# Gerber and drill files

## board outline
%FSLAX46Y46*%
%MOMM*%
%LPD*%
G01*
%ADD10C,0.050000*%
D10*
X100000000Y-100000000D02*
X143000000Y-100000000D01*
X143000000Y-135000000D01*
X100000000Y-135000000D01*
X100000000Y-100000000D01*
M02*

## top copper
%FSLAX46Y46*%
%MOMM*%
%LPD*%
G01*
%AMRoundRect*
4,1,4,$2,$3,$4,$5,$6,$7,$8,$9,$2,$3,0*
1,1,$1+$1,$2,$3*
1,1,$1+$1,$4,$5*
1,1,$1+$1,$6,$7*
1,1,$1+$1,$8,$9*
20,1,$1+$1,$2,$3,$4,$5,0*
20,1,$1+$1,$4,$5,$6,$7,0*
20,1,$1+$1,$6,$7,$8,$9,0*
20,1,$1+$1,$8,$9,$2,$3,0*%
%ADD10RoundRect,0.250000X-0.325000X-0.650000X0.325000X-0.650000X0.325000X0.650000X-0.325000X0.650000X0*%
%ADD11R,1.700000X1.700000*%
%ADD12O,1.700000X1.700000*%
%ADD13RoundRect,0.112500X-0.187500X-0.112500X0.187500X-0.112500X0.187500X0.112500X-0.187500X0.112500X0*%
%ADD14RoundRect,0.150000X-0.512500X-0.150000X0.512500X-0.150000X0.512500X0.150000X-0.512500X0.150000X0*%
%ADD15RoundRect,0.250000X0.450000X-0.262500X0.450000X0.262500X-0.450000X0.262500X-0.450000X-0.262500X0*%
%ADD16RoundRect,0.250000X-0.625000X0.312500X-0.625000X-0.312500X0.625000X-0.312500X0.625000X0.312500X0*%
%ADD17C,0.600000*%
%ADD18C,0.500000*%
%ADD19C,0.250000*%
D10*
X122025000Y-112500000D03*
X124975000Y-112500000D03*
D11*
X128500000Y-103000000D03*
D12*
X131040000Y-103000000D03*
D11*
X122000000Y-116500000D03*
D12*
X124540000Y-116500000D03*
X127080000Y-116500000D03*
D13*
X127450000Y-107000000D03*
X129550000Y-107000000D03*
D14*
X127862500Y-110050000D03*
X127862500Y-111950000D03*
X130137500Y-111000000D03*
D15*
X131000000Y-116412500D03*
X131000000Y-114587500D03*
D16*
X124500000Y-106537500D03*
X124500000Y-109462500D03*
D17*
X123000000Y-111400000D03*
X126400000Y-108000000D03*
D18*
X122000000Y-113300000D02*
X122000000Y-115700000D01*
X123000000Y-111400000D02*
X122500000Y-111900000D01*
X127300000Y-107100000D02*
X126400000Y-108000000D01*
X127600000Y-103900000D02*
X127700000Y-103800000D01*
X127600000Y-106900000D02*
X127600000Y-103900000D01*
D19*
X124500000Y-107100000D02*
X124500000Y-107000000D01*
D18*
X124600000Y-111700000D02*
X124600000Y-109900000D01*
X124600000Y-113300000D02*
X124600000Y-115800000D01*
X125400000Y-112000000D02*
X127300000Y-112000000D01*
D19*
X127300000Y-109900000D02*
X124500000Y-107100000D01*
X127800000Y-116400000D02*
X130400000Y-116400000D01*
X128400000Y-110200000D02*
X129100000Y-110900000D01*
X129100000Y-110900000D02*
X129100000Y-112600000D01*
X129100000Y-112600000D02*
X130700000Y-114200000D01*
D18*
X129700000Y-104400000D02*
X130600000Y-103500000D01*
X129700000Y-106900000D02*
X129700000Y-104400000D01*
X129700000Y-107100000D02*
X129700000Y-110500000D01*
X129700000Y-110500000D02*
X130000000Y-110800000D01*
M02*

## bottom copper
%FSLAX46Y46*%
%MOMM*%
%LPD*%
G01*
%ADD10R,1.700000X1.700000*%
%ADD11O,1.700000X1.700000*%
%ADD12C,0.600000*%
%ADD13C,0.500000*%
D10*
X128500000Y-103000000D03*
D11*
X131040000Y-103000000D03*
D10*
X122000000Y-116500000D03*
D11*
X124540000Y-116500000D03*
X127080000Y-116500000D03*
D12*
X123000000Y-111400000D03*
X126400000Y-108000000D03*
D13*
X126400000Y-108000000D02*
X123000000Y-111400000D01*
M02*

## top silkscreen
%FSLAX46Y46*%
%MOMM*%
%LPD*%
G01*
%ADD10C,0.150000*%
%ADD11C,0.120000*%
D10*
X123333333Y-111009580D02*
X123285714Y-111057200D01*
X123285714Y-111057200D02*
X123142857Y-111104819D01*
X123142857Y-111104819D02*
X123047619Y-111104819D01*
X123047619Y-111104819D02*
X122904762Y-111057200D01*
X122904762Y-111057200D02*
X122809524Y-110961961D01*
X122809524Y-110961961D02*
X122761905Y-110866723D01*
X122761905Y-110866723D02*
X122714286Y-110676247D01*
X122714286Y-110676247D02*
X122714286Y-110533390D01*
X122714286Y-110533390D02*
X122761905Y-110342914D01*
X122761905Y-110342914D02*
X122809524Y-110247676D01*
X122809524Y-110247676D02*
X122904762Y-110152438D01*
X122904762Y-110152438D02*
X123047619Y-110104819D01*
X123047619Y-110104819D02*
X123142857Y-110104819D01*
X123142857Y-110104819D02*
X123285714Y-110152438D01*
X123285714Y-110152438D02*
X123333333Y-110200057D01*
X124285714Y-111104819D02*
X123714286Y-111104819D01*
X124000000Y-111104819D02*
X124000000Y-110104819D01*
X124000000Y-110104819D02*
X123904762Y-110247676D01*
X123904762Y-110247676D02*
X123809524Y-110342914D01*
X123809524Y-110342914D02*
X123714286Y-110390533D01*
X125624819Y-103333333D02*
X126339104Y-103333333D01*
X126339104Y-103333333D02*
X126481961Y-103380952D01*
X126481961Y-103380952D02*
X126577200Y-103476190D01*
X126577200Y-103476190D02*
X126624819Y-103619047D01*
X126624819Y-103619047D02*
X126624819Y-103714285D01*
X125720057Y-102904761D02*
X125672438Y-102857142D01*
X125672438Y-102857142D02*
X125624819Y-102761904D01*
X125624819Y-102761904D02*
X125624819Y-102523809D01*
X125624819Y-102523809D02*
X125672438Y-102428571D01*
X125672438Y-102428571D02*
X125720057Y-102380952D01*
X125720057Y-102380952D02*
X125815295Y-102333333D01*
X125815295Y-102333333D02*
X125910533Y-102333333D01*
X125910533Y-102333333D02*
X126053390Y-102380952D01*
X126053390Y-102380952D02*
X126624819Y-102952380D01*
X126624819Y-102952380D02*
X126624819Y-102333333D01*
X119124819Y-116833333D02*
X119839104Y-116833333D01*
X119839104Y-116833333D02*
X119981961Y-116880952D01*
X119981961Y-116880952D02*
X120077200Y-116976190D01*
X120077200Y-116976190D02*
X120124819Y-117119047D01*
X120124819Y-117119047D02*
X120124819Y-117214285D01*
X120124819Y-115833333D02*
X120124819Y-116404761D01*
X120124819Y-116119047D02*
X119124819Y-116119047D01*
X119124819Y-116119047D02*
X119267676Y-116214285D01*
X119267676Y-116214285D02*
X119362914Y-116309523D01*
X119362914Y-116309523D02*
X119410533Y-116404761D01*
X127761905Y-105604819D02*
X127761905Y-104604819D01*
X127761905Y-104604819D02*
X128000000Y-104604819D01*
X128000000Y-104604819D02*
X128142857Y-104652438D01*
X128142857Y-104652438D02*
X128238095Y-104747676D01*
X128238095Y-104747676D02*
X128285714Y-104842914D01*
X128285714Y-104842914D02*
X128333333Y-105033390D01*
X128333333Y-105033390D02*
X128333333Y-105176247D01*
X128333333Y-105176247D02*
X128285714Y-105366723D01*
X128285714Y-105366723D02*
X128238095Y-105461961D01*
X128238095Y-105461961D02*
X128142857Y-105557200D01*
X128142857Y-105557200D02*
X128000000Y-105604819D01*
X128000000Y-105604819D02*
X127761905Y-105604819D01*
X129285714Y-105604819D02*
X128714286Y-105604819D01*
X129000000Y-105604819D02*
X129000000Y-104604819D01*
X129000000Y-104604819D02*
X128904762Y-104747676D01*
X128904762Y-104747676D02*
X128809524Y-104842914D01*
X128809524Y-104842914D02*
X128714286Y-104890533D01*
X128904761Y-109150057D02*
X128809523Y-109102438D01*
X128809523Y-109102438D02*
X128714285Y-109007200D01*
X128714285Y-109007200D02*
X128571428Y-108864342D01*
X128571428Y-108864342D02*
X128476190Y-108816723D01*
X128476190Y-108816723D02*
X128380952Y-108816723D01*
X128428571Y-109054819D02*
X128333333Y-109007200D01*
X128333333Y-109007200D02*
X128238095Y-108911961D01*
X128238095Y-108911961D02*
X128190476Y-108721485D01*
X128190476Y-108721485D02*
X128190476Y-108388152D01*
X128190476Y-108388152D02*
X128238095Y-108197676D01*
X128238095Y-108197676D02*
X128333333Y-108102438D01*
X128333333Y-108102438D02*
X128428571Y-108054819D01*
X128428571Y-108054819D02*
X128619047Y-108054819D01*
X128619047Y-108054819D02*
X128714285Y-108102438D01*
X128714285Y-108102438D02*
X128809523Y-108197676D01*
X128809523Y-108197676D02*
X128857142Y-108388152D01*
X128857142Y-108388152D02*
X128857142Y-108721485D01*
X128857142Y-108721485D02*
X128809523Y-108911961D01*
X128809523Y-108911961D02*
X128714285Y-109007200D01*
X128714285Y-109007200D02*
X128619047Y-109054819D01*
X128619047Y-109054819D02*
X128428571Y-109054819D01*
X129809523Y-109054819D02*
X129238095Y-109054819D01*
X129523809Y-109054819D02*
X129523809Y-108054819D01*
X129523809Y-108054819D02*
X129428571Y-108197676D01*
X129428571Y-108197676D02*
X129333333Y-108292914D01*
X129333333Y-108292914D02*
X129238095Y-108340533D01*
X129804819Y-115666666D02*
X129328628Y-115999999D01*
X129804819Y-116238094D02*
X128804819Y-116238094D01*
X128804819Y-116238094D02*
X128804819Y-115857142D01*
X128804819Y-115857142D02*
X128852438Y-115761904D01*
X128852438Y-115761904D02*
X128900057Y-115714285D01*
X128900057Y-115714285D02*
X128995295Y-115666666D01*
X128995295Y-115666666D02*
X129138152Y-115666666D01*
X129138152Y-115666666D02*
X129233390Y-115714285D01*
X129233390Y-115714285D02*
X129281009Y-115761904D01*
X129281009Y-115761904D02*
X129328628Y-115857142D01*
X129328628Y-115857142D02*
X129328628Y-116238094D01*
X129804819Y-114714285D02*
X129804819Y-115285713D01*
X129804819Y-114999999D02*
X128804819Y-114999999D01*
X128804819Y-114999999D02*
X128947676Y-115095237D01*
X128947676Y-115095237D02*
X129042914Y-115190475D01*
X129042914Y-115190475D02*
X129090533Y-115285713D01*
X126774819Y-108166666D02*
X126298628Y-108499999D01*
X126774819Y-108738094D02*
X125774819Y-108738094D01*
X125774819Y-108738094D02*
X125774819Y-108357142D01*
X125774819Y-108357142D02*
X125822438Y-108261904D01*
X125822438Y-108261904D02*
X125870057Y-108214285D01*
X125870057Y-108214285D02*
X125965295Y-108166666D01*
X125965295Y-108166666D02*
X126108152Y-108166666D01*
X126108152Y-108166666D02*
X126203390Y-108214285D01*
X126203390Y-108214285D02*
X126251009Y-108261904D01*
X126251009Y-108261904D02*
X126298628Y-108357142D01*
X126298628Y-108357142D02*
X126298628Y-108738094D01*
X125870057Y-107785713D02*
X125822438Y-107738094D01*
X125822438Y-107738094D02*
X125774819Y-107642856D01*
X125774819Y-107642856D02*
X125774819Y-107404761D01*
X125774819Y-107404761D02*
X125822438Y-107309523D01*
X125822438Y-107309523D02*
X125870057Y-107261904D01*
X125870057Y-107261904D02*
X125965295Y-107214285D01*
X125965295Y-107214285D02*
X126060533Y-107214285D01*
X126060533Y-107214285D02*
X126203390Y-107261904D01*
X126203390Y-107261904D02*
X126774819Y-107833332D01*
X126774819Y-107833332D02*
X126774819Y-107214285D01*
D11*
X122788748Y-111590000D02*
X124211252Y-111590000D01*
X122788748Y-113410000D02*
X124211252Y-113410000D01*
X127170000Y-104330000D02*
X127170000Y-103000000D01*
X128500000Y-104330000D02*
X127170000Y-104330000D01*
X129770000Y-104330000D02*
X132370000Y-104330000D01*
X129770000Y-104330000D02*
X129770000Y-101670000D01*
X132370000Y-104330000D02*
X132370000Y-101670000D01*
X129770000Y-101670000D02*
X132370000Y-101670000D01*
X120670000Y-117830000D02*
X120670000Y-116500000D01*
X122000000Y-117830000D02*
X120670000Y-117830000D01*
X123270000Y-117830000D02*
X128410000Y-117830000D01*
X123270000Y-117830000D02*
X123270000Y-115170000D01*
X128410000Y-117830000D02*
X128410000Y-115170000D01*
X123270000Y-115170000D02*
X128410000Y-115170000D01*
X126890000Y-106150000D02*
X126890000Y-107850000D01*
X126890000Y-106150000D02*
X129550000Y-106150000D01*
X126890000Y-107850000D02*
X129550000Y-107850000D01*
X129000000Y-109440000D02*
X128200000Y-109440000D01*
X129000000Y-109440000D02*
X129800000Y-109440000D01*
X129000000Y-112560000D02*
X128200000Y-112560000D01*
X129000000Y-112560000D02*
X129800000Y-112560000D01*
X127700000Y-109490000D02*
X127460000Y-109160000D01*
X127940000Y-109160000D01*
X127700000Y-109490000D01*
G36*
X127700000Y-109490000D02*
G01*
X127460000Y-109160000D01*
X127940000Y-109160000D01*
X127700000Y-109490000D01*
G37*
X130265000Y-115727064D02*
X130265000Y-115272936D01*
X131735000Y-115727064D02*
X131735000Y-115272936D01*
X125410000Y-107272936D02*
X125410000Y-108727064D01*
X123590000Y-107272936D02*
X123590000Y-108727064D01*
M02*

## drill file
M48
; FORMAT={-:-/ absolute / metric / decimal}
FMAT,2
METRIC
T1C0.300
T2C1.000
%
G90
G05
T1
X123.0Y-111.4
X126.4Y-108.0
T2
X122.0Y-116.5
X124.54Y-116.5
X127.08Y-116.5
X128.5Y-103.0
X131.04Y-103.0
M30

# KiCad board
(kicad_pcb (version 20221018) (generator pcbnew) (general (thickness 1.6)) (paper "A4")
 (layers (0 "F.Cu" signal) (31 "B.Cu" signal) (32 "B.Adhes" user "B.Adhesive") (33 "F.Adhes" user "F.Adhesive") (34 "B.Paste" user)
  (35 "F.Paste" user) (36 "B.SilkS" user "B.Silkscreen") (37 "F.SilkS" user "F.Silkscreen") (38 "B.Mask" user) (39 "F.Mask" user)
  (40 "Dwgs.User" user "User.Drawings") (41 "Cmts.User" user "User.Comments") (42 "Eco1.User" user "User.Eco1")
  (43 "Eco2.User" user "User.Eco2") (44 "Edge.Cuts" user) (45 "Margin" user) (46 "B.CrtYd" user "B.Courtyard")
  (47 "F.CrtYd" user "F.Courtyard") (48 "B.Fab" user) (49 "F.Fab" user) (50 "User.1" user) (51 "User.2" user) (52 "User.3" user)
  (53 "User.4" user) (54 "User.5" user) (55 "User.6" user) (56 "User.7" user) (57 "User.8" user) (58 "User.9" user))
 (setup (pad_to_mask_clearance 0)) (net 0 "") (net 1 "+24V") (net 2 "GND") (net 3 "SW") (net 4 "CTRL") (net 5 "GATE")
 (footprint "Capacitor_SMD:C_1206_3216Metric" (layer "F.Cu") (at 123.5 112.5)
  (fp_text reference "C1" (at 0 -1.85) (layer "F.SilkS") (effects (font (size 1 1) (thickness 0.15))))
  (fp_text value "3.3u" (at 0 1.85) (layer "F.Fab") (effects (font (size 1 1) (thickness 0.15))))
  (fp_line (start -0.711252 -0.91) (end 0.711252 -0.91) (stroke (width 0.12) (type solid)) (layer "F.SilkS"))
  (fp_line (start -0.711252 0.91) (end 0.711252 0.91) (stroke (width 0.12) (type solid)) (layer "F.SilkS"))
  (pad "1" smd roundrect (at -1.475 0) (size 1.15 1.8) (layers "F.Cu" "F.Paste" "F.Mask") (roundrect_rratio 0.217391) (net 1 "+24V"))
  (pad "2" smd roundrect (at 1.475 0) (size 1.15 1.8) (layers "F.Cu" "F.Paste" "F.Mask") (roundrect_rratio 0.217391) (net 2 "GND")))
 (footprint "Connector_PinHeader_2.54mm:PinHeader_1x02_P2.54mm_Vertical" (layer "F.Cu") (at 128.5 103 90)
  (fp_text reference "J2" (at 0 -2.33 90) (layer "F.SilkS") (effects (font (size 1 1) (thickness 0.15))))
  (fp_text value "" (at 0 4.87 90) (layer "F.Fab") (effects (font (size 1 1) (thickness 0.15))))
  (fp_line (start -1.33 -1.33) (end 0 -1.33) (stroke (width 0.12) (type solid)) (layer "F.SilkS"))
  (fp_line (start -1.33 0) (end -1.33 -1.33) (stroke (width 0.12) (type solid)) (layer "F.SilkS"))
  (fp_line (start -1.33 1.27) (end -1.33 3.87) (stroke (width 0.12) (type solid)) (layer "F.SilkS"))
  (fp_line (start -1.33 1.27) (end 1.33 1.27) (stroke (width 0.12) (type solid)) (layer "F.SilkS"))
  (fp_line (start -1.33 3.87) (end 1.33 3.87) (stroke (width 0.12) (type solid)) (layer "F.SilkS"))
  (fp_line (start 1.33 1.27) (end 1.33 3.87) (stroke (width 0.12) (type solid)) (layer "F.SilkS"))
  (pad "1" thru_hole rect (at 0 0 90) (size 1.7 1.7) (drill 1) (layers "*.Cu" "*.Mask") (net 1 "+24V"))
  (pad "2" thru_hole oval (at 0 2.54 90) (size 1.7 1.7) (drill 1) (layers "*.Cu" "*.Mask") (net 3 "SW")))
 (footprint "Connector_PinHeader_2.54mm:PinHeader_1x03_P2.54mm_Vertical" (layer "F.Cu") (at 122 116.5 90)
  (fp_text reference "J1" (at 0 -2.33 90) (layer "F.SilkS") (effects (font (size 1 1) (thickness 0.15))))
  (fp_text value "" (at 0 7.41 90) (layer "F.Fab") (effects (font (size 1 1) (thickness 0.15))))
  (fp_line (start -1.33 -1.33) (end 0 -1.33) (stroke (width 0.12) (type solid)) (layer "F.SilkS"))
  (fp_line (start -1.33 0) (end -1.33 -1.33) (stroke (width 0.12) (type solid)) (layer "F.SilkS"))
  (fp_line (start -1.33 1.27) (end -1.33 6.41) (stroke (width 0.12) (type solid)) (layer "F.SilkS"))
  (fp_line (start -1.33 1.27) (end 1.33 1.27) (stroke (width 0.12) (type solid)) (layer "F.SilkS"))
  (fp_line (start -1.33 6.41) (end 1.33 6.41) (stroke (width 0.12) (type solid)) (layer "F.SilkS"))
  (fp_line (start 1.33 1.27) (end 1.33 6.41) (stroke (width 0.12) (type solid)) (layer "F.SilkS"))
  (pad "1" thru_hole rect (at 0 0 90) (size 1.7 1.7) (drill 1) (layers "*.Cu" "*.Mask") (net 1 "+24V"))
  (pad "2" thru_hole oval (at 0 2.54 90) (size 1.7 1.7) (drill 1) (layers "*.Cu" "*.Mask") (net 2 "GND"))
  (pad "3" thru_hole oval (at 0 5.08 90) (size 1.7 1.7) (drill 1) (layers "*.Cu" "*.Mask") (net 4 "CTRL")))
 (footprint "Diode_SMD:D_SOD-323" (layer "F.Cu") (at 128.5 107)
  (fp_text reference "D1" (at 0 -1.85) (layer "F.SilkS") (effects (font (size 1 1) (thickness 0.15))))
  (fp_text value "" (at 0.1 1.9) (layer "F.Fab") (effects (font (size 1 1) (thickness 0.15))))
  (fp_line (start -1.61 -0.85) (end -1.61 0.85) (stroke (width 0.12) (type solid)) (layer "F.SilkS"))
  (fp_line (start -1.61 -0.85) (end 1.05 -0.85) (stroke (width 0.12) (type solid)) (layer "F.SilkS"))
  (fp_line (start -1.61 0.85) (end 1.05 0.85) (stroke (width 0.12) (type solid)) (layer "F.SilkS"))
  (pad "1" smd roundrect (at -1.05 0) (size 0.6 0.45) (layers "F.Cu" "F.Paste" "F.Mask") (roundrect_rratio 0.25) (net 1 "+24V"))
  (pad "2" smd roundrect (at 1.05 0) (size 0.6 0.45) (layers "F.Cu" "F.Paste" "F.Mask") (roundrect_rratio 0.25) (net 3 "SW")))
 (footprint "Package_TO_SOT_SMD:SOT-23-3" (layer "F.Cu") (at 129 111)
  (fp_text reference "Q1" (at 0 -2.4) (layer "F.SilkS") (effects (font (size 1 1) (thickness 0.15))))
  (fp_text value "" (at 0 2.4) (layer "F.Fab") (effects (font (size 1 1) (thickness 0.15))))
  (fp_line (start 0 -1.56) (end -0.8 -1.56) (stroke (width 0.12) (type solid)) (layer "F.SilkS"))
  (fp_line (start 0 -1.56) (end 0.8 -1.56) (stroke (width 0.12) (type solid)) (layer "F.SilkS"))
  (fp_line (start 0 1.56) (end -0.8 1.56) (stroke (width 0.12) (type solid)) (layer "F.SilkS"))
  (fp_line (start 0 1.56) (end 0.8 1.56) (stroke (width 0.12) (type solid)) (layer "F.SilkS"))
  (fp_poly
   (pts (xy -1.3 -1.51) (xy -1.54 -1.84) (xy -1.06 -1.84) (xy -1.3 -1.51)) (stroke (width 0.12) (type solid)) (fill solid) (layer "F.SilkS"))
  (pad "1" smd roundrect (at -1.1375 -0.95) (size 1.325 0.6) (layers "F.Cu" "F.Paste" "F.Mask") (roundrect_rratio 0.25) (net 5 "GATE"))
  (pad "2" smd roundrect (at -1.1375 0.95) (size 1.325 0.6) (layers "F.Cu" "F.Paste" "F.Mask") (roundrect_rratio 0.25) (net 2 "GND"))
  (pad "3" smd roundrect (at 1.1375 0) (size 1.325 0.6) (layers "F.Cu" "F.Paste" "F.Mask") (roundrect_rratio 0.25) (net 3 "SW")))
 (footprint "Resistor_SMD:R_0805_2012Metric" (layer "F.Cu") (at 131 115.5 90)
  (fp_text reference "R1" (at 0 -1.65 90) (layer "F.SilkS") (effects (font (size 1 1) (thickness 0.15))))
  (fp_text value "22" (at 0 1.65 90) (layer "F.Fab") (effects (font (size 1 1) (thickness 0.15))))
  (fp_line (start -0.227064 -0.735) (end 0.227064 -0.735) (stroke (width 0.12) (type solid)) (layer "F.SilkS"))
  (fp_line (start -0.227064 0.735) (end 0.227064 0.735) (stroke (width 0.12) (type solid)) (layer "F.SilkS"))
  (pad "1" smd roundrect (at -0.9125 0 90) (size 1.025 1.4) (layers "F.Cu" "F.Paste" "F.Mask") (roundrect_rratio 0.243902) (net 4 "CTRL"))
  (pad "2" smd roundrect (at 0.9125 0 90) (size 1.025 1.4) (layers "F.Cu" "F.Paste" "F.Mask") (roundrect_rratio 0.243902) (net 5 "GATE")))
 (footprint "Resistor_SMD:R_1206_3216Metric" (layer "F.Cu") (at 124.5 108 -90)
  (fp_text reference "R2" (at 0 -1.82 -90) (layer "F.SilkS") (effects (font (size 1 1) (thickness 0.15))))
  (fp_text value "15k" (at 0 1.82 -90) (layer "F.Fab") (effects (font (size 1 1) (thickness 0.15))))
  (fp_line (start -0.727064 -0.91) (end 0.727064 -0.91) (stroke (width 0.12) (type solid)) (layer "F.SilkS"))
  (fp_line (start -0.727064 0.91) (end 0.727064 0.91) (stroke (width 0.12) (type solid)) (layer "F.SilkS"))
  (pad "1" smd roundrect (at -1.4625 0 270) (size 1.125 1.75) (layers "F.Cu" "F.Paste" "F.Mask") (roundrect_rratio 0.222222) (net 5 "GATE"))
  (pad "2" smd roundrect (at 1.4625 0 270) (size 1.125 1.75) (layers "F.Cu" "F.Paste" "F.Mask") (roundrect_rratio 0.222222) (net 2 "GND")))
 (gr_rect (start 100 100) (end 143 135) (stroke (width 0.05) (type default)) (fill none) (layer "Edge.Cuts"))
 (segment (start 122 113.3) (end 122 115.7) (width 0.5) (layer "F.Cu") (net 1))
 (segment (start 123 111.4) (end 122.5 111.9) (width 0.5) (layer "F.Cu") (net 1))
 (segment (start 127.3 107.1) (end 126.4 108) (width 0.5) (layer "F.Cu") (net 1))
 (segment (start 127.6 103.9) (end 127.7 103.8) (width 0.5) (layer "F.Cu") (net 1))
 (segment (start 127.6 106.9) (end 127.6 103.9) (width 0.5) (layer "F.Cu") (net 1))
 (via (at 123 111.4) (size 0.6) (drill 0.3) (layers "F.Cu" "B.Cu") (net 1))
 (via (at 126.4 108) (size 0.6) (drill 0.3) (layers "F.Cu" "B.Cu") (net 1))
 (segment (start 124.5 107.1) (end 124.5 107) (width 0.25) (layer "F.Cu") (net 5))
 (segment (start 124.6 111.7) (end 124.6 109.9) (width 0.5) (layer "F.Cu") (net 2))
 (segment (start 124.6 113.3) (end 124.6 115.8) (width 0.5) (layer "F.Cu") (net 2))
 (segment (start 125.4 112) (end 127.3 112) (width 0.5) (layer "F.Cu") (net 2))
 (segment (start 126.4 108) (end 123 111.4) (width 0.5) (layer "B.Cu") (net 1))
 (segment (start 127.3 109.9) (end 124.5 107.1) (width 0.25) (layer "F.Cu") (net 5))
 (segment (start 127.8 116.4) (end 130.4 116.4) (width 0.25) (layer "F.Cu") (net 4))
 (segment (start 128.4 110.2) (end 129.1 110.9) (width 0.25) (layer "F.Cu") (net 5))
 (segment (start 129.1 110.9) (end 129.1 112.6) (width 0.25) (layer "F.Cu") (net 5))
 (segment (start 129.1 112.6) (end 130.7 114.2) (width 0.25) (layer "F.Cu") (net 5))
 (segment (start 129.7 104.4) (end 130.6 103.5) (width 0.5) (layer "F.Cu") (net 3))
 (segment (start 129.7 106.9) (end 129.7 104.4) (width 0.5) (layer "F.Cu") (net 3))
 (segment (start 129.7 107.1) (end 129.7 110.5) (width 0.5) (layer "F.Cu") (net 3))
 (segment (start 129.7 110.5) (end 130 110.8) (width 0.5) (layer "F.Cu") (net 3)))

